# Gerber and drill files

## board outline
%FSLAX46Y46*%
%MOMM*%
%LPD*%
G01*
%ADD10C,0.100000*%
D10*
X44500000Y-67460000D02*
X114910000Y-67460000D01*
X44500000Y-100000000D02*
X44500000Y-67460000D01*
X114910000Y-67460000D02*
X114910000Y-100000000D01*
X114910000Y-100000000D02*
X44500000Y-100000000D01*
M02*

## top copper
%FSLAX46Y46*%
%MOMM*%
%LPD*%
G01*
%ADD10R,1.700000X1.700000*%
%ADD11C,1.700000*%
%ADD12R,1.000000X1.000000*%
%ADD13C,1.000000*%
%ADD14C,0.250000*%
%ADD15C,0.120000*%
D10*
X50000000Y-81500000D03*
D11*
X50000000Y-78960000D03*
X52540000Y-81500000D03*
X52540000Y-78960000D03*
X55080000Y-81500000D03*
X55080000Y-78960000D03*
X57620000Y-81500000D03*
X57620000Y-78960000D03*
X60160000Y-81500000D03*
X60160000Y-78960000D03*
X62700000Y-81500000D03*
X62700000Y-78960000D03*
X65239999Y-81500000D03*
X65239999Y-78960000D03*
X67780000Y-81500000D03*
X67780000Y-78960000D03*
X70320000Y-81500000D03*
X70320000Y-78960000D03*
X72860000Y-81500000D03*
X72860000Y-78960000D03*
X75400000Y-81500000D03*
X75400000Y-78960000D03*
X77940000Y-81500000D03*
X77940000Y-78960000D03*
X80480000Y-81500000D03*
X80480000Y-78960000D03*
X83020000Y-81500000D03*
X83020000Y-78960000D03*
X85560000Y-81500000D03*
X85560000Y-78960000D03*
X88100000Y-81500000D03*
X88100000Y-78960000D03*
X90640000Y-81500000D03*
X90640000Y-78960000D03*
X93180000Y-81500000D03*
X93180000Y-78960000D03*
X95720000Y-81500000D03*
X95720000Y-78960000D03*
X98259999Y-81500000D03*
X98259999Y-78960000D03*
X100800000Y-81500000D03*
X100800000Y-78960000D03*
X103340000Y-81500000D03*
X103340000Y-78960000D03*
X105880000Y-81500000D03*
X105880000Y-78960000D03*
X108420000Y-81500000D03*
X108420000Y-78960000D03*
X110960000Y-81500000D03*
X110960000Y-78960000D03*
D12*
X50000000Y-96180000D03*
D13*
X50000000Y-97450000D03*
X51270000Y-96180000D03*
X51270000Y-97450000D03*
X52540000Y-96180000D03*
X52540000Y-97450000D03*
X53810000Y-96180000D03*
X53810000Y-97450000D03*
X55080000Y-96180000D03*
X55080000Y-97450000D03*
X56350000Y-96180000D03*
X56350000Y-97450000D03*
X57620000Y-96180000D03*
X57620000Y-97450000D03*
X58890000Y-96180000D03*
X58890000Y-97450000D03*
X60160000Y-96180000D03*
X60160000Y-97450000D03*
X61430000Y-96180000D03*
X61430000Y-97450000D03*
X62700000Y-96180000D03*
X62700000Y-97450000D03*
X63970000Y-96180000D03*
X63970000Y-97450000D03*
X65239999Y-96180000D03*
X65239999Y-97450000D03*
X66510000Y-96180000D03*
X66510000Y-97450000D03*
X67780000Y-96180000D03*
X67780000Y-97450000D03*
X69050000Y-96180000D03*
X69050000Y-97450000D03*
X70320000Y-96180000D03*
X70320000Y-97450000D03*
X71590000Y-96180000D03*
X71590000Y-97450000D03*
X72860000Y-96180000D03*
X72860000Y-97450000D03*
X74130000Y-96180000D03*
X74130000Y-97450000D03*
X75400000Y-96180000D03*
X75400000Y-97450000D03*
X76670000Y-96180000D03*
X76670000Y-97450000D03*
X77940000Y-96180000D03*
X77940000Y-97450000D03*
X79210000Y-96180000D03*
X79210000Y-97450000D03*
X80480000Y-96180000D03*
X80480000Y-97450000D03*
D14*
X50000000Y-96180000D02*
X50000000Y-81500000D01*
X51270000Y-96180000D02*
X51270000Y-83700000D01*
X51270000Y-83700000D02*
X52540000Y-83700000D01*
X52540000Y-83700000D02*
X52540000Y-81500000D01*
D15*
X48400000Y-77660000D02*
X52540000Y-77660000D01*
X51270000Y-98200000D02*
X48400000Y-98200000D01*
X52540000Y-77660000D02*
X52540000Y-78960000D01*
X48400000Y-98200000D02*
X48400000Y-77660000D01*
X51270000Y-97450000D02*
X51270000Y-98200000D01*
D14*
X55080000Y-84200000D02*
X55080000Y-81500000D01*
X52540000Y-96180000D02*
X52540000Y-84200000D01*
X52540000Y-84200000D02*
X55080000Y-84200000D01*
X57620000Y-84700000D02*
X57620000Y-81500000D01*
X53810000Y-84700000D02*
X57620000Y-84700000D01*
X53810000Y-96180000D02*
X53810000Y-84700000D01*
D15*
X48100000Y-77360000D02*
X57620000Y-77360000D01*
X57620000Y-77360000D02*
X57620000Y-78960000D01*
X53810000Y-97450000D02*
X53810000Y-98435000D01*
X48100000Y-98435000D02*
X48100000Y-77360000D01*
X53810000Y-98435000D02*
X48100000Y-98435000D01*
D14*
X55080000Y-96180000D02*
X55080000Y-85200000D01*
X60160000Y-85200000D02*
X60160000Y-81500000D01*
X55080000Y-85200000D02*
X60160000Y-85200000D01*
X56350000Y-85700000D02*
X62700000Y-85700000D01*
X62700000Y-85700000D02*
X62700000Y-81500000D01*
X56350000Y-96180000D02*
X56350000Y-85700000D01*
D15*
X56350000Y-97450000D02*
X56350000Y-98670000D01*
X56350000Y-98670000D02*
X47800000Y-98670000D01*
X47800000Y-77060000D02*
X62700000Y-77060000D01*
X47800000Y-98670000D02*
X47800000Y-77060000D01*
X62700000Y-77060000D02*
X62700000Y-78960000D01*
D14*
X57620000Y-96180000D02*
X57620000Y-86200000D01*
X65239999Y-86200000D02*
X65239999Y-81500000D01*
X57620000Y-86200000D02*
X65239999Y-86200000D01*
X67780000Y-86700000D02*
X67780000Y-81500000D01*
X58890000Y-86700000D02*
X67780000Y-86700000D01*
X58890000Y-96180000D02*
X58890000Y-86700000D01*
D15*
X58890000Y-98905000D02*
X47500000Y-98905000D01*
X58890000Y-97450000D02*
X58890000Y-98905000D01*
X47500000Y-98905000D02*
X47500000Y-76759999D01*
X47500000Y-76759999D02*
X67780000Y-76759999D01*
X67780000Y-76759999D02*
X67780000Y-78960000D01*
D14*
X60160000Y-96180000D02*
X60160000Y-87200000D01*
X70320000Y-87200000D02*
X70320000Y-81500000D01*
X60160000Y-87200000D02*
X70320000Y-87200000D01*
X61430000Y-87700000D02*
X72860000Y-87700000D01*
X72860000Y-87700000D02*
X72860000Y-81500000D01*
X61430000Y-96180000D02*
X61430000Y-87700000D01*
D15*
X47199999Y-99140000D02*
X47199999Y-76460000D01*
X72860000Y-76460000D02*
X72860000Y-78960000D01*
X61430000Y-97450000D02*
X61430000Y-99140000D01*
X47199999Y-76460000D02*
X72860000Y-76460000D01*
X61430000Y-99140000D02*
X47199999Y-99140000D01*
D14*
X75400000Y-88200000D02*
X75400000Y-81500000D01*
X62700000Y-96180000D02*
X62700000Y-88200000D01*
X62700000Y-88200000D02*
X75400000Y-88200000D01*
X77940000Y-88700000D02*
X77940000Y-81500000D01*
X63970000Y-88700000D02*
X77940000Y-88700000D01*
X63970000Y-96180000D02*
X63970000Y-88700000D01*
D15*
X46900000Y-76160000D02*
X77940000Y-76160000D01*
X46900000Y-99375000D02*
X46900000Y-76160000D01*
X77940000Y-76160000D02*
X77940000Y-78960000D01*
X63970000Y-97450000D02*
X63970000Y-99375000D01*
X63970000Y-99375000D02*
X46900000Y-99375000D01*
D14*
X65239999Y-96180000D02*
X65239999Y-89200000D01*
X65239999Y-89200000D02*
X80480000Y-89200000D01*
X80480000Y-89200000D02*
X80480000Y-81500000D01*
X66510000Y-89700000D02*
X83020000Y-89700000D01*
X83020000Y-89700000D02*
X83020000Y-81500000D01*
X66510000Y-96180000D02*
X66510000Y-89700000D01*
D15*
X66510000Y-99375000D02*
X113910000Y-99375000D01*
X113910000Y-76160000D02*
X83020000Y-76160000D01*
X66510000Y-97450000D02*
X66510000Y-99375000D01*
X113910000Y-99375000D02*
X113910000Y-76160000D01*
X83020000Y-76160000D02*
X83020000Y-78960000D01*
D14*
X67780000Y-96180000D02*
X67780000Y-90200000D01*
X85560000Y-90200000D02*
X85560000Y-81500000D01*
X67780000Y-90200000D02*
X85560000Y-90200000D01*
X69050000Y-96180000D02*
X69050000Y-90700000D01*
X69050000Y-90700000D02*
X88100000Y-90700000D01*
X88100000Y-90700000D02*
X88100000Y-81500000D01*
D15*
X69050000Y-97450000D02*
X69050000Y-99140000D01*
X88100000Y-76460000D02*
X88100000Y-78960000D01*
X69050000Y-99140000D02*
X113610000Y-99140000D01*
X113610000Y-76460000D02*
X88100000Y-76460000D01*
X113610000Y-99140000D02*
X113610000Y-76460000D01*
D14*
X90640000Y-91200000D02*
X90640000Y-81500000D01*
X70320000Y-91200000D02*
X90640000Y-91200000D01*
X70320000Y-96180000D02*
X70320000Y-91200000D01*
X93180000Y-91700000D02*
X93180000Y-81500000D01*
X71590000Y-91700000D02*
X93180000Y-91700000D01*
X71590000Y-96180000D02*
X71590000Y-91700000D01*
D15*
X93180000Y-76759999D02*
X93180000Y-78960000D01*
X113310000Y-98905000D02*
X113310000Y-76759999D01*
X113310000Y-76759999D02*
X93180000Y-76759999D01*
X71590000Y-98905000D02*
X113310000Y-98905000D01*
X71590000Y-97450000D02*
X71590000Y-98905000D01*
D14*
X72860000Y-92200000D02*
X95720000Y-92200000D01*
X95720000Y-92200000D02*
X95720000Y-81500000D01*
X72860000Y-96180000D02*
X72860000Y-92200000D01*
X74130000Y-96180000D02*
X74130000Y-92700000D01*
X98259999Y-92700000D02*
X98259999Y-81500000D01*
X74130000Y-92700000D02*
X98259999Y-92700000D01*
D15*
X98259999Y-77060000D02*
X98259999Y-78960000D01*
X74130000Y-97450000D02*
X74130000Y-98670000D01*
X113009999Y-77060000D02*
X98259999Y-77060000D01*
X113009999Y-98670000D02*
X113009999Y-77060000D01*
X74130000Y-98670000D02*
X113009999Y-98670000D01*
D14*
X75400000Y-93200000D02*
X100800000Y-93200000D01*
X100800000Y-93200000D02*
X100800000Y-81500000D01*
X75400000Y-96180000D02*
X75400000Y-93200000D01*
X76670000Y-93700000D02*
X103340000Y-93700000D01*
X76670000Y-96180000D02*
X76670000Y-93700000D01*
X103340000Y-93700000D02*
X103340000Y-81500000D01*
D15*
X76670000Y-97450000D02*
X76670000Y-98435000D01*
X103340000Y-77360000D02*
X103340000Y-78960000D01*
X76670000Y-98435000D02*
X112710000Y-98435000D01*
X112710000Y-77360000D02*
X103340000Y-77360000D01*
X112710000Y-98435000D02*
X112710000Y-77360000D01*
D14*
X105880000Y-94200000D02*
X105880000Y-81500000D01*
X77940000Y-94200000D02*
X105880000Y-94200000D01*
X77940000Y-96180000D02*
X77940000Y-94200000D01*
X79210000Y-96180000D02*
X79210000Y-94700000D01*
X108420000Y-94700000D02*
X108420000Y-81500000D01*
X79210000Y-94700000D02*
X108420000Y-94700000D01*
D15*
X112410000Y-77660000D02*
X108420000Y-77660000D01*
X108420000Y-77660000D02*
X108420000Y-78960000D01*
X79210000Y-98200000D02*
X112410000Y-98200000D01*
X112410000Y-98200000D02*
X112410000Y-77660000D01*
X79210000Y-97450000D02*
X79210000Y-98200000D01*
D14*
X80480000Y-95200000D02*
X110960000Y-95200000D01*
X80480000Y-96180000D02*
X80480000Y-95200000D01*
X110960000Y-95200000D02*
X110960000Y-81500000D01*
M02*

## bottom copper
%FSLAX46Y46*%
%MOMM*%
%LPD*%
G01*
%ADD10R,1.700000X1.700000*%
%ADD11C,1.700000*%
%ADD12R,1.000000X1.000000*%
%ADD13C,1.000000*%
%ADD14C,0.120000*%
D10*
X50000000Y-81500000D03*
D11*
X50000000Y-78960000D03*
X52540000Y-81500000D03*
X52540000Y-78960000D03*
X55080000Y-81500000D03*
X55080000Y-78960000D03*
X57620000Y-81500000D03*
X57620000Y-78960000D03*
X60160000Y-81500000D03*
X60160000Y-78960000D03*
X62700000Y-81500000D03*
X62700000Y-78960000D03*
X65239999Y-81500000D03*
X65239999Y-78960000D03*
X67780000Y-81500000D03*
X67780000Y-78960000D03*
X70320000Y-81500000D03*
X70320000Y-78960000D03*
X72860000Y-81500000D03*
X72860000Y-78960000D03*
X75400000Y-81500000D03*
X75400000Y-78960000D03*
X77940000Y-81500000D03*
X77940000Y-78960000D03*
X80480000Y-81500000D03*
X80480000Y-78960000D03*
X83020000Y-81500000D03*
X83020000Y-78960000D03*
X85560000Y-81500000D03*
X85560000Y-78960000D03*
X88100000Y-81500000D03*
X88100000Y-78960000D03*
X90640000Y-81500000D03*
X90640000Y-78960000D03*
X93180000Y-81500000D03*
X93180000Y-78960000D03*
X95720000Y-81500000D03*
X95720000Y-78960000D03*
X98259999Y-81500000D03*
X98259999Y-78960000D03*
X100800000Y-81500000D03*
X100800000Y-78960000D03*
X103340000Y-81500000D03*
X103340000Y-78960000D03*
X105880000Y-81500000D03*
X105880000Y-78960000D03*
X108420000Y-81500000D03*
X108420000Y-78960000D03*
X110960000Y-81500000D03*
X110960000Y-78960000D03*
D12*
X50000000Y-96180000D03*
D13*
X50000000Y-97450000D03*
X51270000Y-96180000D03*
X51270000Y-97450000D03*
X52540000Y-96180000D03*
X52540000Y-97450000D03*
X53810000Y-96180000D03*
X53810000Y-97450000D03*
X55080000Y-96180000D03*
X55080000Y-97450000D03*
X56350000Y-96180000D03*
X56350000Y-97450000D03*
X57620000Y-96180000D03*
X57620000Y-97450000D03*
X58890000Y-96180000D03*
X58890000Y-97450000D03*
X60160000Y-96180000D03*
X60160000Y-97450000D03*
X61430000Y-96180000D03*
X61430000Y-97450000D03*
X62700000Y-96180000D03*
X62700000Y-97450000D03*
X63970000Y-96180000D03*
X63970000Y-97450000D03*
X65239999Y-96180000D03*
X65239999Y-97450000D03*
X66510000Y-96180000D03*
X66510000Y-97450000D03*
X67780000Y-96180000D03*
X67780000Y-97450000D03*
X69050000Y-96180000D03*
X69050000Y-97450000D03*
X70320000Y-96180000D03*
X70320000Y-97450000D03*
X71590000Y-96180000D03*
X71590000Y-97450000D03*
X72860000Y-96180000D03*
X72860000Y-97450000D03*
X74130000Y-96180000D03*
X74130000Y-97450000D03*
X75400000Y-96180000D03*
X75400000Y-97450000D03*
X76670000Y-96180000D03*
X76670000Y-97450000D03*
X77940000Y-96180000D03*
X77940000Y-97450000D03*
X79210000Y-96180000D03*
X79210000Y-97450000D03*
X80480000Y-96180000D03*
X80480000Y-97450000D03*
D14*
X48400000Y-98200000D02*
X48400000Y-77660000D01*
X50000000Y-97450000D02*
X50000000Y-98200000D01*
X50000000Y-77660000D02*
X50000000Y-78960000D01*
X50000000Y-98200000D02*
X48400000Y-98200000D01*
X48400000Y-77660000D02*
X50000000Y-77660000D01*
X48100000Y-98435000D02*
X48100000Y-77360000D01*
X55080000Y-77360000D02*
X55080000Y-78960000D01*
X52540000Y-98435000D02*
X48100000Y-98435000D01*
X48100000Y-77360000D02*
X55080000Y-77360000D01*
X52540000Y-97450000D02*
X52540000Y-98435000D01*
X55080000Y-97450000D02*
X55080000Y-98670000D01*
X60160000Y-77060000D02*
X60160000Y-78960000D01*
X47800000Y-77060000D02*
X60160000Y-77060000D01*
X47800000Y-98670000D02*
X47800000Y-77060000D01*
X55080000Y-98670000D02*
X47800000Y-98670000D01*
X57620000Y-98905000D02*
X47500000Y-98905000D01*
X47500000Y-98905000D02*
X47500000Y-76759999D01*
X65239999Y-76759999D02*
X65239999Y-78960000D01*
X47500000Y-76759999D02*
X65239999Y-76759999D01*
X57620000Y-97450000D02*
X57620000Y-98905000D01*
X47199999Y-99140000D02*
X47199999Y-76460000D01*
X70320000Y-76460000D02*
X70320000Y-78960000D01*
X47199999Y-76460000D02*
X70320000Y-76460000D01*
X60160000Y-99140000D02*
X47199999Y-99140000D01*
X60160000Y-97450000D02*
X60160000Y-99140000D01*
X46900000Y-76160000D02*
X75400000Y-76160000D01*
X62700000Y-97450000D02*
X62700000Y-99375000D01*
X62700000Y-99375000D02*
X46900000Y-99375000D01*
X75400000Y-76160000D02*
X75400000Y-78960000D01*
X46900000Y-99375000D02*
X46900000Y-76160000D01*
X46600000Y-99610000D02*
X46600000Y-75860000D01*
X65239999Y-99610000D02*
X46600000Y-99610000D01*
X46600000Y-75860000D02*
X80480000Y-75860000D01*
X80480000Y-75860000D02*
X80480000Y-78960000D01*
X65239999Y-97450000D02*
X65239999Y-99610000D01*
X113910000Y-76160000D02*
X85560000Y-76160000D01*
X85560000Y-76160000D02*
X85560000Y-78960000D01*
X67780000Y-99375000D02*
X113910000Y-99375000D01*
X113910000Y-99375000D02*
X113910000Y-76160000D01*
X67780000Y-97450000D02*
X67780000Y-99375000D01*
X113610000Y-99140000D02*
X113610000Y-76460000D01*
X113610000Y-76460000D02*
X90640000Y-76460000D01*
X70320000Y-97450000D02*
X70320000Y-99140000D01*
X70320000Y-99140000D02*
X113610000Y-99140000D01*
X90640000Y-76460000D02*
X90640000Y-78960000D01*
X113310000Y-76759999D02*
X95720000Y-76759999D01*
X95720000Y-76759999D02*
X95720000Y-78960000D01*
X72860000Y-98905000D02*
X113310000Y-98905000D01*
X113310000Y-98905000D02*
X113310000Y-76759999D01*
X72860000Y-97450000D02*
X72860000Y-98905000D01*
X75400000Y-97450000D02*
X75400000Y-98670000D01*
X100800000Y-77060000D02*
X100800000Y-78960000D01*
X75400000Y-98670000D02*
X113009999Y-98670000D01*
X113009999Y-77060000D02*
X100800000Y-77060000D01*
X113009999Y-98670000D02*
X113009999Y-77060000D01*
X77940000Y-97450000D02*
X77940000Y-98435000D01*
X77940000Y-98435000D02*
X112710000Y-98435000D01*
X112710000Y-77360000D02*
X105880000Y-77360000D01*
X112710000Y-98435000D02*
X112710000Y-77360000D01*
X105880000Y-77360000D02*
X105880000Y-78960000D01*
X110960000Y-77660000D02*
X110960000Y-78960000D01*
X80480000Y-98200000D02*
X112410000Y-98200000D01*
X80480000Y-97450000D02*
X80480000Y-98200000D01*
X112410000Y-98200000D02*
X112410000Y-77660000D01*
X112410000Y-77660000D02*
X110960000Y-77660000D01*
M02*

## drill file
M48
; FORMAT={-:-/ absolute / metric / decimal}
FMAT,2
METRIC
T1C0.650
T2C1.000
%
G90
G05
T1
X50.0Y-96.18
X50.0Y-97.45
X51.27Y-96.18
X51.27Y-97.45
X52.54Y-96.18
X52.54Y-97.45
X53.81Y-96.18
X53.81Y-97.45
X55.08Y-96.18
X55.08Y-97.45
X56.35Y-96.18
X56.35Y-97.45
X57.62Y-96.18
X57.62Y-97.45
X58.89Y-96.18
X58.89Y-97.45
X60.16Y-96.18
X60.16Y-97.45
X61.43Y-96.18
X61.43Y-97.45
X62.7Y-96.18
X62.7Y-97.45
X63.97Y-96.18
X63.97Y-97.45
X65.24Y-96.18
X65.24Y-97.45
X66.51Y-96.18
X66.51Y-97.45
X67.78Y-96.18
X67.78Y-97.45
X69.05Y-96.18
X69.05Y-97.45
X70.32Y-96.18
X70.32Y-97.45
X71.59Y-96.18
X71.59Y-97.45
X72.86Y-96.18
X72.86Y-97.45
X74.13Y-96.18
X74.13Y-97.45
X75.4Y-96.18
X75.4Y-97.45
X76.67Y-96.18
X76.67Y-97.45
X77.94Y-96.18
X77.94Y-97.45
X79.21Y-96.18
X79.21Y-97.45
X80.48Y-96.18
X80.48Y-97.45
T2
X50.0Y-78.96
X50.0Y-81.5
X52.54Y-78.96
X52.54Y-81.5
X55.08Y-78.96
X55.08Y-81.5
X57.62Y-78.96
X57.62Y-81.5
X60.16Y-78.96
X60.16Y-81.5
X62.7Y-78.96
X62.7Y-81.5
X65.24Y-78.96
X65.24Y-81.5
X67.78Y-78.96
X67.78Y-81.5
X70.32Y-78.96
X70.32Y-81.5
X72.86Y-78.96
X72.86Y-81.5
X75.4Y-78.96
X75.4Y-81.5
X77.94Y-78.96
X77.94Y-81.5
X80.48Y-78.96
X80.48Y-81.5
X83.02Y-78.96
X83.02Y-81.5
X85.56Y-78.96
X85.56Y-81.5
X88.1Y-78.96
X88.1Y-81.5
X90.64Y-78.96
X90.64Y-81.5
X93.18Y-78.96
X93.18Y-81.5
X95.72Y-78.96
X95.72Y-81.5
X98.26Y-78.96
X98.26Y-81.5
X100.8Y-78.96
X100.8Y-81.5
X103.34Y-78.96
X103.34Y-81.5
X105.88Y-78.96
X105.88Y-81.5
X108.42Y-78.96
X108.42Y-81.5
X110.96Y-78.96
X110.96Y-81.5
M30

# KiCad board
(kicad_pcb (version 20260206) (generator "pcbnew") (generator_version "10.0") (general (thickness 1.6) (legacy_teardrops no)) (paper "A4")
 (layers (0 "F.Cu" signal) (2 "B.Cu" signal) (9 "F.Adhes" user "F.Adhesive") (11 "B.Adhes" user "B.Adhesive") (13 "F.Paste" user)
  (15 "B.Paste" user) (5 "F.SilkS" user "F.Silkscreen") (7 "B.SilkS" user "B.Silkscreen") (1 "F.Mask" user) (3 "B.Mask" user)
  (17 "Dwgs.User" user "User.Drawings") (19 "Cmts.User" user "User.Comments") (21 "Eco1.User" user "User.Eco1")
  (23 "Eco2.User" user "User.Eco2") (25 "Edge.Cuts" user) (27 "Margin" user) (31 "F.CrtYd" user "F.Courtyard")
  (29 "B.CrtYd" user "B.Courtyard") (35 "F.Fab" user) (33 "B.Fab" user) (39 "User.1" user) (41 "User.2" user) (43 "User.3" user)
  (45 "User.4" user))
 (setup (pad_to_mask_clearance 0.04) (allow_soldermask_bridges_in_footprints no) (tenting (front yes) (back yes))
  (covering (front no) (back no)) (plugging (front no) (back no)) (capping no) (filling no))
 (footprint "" (layer "F.Cu") (at 80.48 80.229999)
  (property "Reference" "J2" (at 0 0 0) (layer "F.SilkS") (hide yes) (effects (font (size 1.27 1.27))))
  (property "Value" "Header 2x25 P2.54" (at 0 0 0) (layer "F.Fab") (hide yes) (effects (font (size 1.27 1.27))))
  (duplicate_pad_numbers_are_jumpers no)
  (pad "1" thru_hole rect (at -30.48 1.270001) (size 1.7 1.7) (drill 1) (layers "*.Cu" "*.Mask") (remove_unused_layers no) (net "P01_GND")
   (thermal_bridge_angle 45))
  (pad "2" thru_hole circle (at -30.48 -1.269999) (size 1.7 1.7) (drill 1) (layers "*.Cu" "*.Mask") (remove_unused_layers no) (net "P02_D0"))
  (pad "3" thru_hole circle (at -27.94 1.270001) (size 1.7 1.7) (drill 1) (layers "*.Cu" "*.Mask") (remove_unused_layers no) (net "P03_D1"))
  (pad "4" thru_hole circle (at -27.94 -1.269999) (size 1.7 1.7) (drill 1) (layers "*.Cu" "*.Mask") (remove_unused_layers no) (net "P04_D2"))
  (pad "5" thru_hole circle (at -25.4 1.270001) (size 1.7 1.7) (drill 1) (layers "*.Cu" "*.Mask") (remove_unused_layers no) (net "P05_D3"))
  (pad "6" thru_hole circle (at -25.4 -1.269999) (size 1.7 1.7) (drill 1) (layers "*.Cu" "*.Mask") (remove_unused_layers no) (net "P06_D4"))
  (pad "7" thru_hole circle (at -22.86 1.270001) (size 1.7 1.7) (drill 1) (layers "*.Cu" "*.Mask") (remove_unused_layers no) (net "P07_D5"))
  (pad "8" thru_hole circle (at -22.86 -1.269999) (size 1.7 1.7) (drill 1) (layers "*.Cu" "*.Mask") (remove_unused_layers no) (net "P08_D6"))
  (pad "9" thru_hole circle (at -20.32 1.270001) (size 1.7 1.7) (drill 1) (layers "*.Cu" "*.Mask") (remove_unused_layers no) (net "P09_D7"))
  (pad "10" thru_hole circle (at -20.32 -1.269999) (size 1.7 1.7) (drill 1) (layers "*.Cu" "*.Mask") (remove_unused_layers no)
   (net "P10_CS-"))
  (pad "11" thru_hole circle (at -17.78 1.270001) (size 1.7 1.7) (drill 1) (layers "*.Cu" "*.Mask") (remove_unused_layers no)
   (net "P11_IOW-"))
  (pad "12" thru_hole circle (at -17.78 -1.269999) (size 1.7 1.7) (drill 1) (layers "*.Cu" "*.Mask") (remove_unused_layers no)
   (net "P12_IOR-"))
  (pad "13" thru_hole circle (at -15.240001 1.270001) (size 1.7 1.7) (drill 1) (layers "*.Cu" "*.Mask") (remove_unused_layers no)
   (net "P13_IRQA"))
  (pad "14" thru_hole circle (at -15.240001 -1.269999) (size 1.7 1.7) (drill 1) (layers "*.Cu" "*.Mask") (remove_unused_layers no)
   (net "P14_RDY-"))
  (pad "15" thru_hole circle (at -12.7 1.270001) (size 1.7 1.7) (drill 1) (layers "*.Cu" "*.Mask") (remove_unused_layers no) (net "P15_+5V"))
  (pad "16" thru_hole circle (at -12.7 -1.269999) (size 1.7 1.7) (drill 1) (layers "*.Cu" "*.Mask") (remove_unused_layers no)
   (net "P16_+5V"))
  (pad "17" thru_hole circle (at -10.16 1.270001) (size 1.7 1.7) (drill 1) (layers "*.Cu" "*.Mask") (remove_unused_layers no)
   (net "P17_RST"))
  (pad "18" thru_hole circle (at -10.16 -1.269999) (size 1.7 1.7) (drill 1) (layers "*.Cu" "*.Mask") (remove_unused_layers no)
   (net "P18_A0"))
  (pad "19" thru_hole circle (at -7.62 1.270001) (size 1.7 1.7) (drill 1) (layers "*.Cu" "*.Mask") (remove_unused_layers no) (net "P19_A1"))
  (pad "20" thru_hole circle (at -7.62 -1.269999) (size 1.7 1.7) (drill 1) (layers "*.Cu" "*.Mask") (remove_unused_layers no) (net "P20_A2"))
  (pad "21" thru_hole circle (at -5.08 1.270001) (size 1.7 1.7) (drill 1) (layers "*.Cu" "*.Mask") (remove_unused_layers no) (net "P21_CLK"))
  (pad "22" thru_hole circle (at -5.08 -1.269999) (size 1.7 1.7) (drill 1) (layers "*.Cu" "*.Mask") (remove_unused_layers no)
   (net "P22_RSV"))
  (pad "23" thru_hole circle (at -2.54 1.270001) (size 1.7 1.7) (drill 1) (layers "*.Cu" "*.Mask") (remove_unused_layers no)
   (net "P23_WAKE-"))
  (pad "24" thru_hole circle (at -2.54 -1.269999) (size 1.7 1.7) (drill 1) (layers "*.Cu" "*.Mask") (remove_unused_layers no)
   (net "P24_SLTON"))
  (pad "25" thru_hole circle (at 0 1.270001) (size 1.7 1.7) (drill 1) (layers "*.Cu" "*.Mask") (remove_unused_layers no) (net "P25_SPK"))
  (pad "26" thru_hole circle (at 0 -1.269999) (size 1.7 1.7) (drill 1) (layers "*.Cu" "*.Mask") (remove_unused_layers no) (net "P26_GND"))
  (pad "27" thru_hole circle (at 2.54 1.270001) (size 1.7 1.7) (drill 1) (layers "*.Cu" "*.Mask") (remove_unused_layers no) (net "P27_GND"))
  (pad "28" thru_hole circle (at 2.54 -1.269999) (size 1.7 1.7) (drill 1) (layers "*.Cu" "*.Mask") (remove_unused_layers no) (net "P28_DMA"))
  (pad "29" thru_hole circle (at 5.08 1.270001) (size 1.7 1.7) (drill 1) (layers "*.Cu" "*.Mask") (remove_unused_layers no) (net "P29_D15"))
  (pad "30" thru_hole circle (at 5.08 -1.269999) (size 1.7 1.7) (drill 1) (layers "*.Cu" "*.Mask") (remove_unused_layers no) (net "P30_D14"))
  (pad "31" thru_hole circle (at 7.62 1.270001) (size 1.7 1.7) (drill 1) (layers "*.Cu" "*.Mask") (remove_unused_layers no) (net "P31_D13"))
  (pad "32" thru_hole circle (at 7.62 -1.269999) (size 1.7 1.7) (drill 1) (layers "*.Cu" "*.Mask") (remove_unused_layers no) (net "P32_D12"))
  (pad "33" thru_hole circle (at 10.16 1.270001) (size 1.7 1.7) (drill 1) (layers "*.Cu" "*.Mask") (remove_unused_layers no) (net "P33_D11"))
  (pad "34" thru_hole circle (at 10.16 -1.269999) (size 1.7 1.7) (drill 1) (layers "*.Cu" "*.Mask") (remove_unused_layers no)
   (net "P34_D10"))
  (pad "35" thru_hole circle (at 12.7 1.270001) (size 1.7 1.7) (drill 1) (layers "*.Cu" "*.Mask") (remove_unused_layers no) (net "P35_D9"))
  (pad "36" thru_hole circle (at 12.7 -1.269999) (size 1.7 1.7) (drill 1) (layers "*.Cu" "*.Mask") (remove_unused_layers no) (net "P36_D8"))
  (pad "37" thru_hole circle (at 15.24 1.270001) (size 1.7 1.7) (drill 1) (layers "*.Cu" "*.Mask") (remove_unused_layers no) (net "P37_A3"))
  (pad "38" thru_hole circle (at 15.24 -1.269999) (size 1.7 1.7) (drill 1) (layers "*.Cu" "*.Mask") (remove_unused_layers no) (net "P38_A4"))
  (pad "39" thru_hole circle (at 17.779999 1.270001) (size 1.7 1.7) (drill 1) (layers "*.Cu" "*.Mask") (remove_unused_layers no)
   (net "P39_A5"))
  (pad "40" thru_hole circle (at 17.779999 -1.269999) (size 1.7 1.7) (drill 1) (layers "*.Cu" "*.Mask") (remove_unused_layers no)
   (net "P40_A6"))
  (pad "41" thru_hole circle (at 20.32 1.270001) (size 1.7 1.7) (drill 1) (layers "*.Cu" "*.Mask") (remove_unused_layers no) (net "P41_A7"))
  (pad "42" thru_hole circle (at 20.32 -1.269999) (size 1.7 1.7) (drill 1) (layers "*.Cu" "*.Mask") (remove_unused_layers no) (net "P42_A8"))
  (pad "43" thru_hole circle (at 22.86 1.270001) (size 1.7 1.7) (drill 1) (layers "*.Cu" "*.Mask") (remove_unused_layers no) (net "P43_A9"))
  (pad "44" thru_hole circle (at 22.86 -1.269999) (size 1.7 1.7) (drill 1) (layers "*.Cu" "*.Mask") (remove_unused_layers no)
   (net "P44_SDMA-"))
  (pad "45" thru_hole circle (at 25.4 1.270001) (size 1.7 1.7) (drill 1) (layers "*.Cu" "*.Mask") (remove_unused_layers no) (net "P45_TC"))
  (pad "46" thru_hole circle (at 25.4 -1.269999) (size 1.7 1.7) (drill 1) (layers "*.Cu" "*.Mask") (remove_unused_layers no)
   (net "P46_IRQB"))
  (pad "47" thru_hole circle (at 27.94 1.270001) (size 1.7 1.7) (drill 1) (layers "*.Cu" "*.Mask") (remove_unused_layers no)
   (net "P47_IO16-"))
  (pad "48" thru_hole circle (at 27.94 -1.269999) (size 1.7 1.7) (drill 1) (layers "*.Cu" "*.Mask") (remove_unused_layers no)
   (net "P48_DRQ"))
  (pad "49" thru_hole circle (at 30.48 1.270001) (size 1.7 1.7) (drill 1) (layers "*.Cu" "*.Mask") (remove_unused_layers no)
   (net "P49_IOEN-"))
  (pad "50" thru_hole circle (at 30.48 -1.269999) (size 1.7 1.7) (drill 1) (layers "*.Cu" "*.Mask") (remove_unused_layers no)
   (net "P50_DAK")))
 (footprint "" (layer "F.Cu") (at 65.239999 96.815)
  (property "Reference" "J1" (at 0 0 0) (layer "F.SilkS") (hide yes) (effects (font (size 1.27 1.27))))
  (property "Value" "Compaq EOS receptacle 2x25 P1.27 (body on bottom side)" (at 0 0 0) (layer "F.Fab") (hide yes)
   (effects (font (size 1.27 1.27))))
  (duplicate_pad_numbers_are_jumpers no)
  (pad "1" thru_hole rect (at -15.239999 -0.635) (size 1 1) (drill 0.65) (layers "*.Cu" "*.Mask") (remove_unused_layers no) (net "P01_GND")
   (thermal_bridge_angle 45))
  (pad "2" thru_hole circle (at -15.239999 0.635) (size 1 1) (drill 0.65) (layers "*.Cu" "*.Mask") (remove_unused_layers no) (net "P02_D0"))
  (pad "3" thru_hole circle (at -13.969999 -0.635) (size 1 1) (drill 0.65) (layers "*.Cu" "*.Mask") (remove_unused_layers no) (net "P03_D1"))
  (pad "4" thru_hole circle (at -13.969999 0.635) (size 1 1) (drill 0.65) (layers "*.Cu" "*.Mask") (remove_unused_layers no) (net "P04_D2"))
  (pad "5" thru_hole circle (at -12.699999 -0.635) (size 1 1) (drill 0.65) (layers "*.Cu" "*.Mask") (remove_unused_layers no) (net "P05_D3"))
  (pad "6" thru_hole circle (at -12.699999 0.635) (size 1 1) (drill 0.65) (layers "*.Cu" "*.Mask") (remove_unused_layers no) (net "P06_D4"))
  (pad "7" thru_hole circle (at -11.429999 -0.635) (size 1 1) (drill 0.65) (layers "*.Cu" "*.Mask") (remove_unused_layers no) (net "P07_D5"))
  (pad "8" thru_hole circle (at -11.429999 0.635) (size 1 1) (drill 0.65) (layers "*.Cu" "*.Mask") (remove_unused_layers no) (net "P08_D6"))
  (pad "9" thru_hole circle (at -10.159999 -0.635) (size 1 1) (drill 0.65) (layers "*.Cu" "*.Mask") (remove_unused_layers no) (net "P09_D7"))
  (pad "10" thru_hole circle (at -10.159999 0.635) (size 1 1) (drill 0.65) (layers "*.Cu" "*.Mask") (remove_unused_layers no)
   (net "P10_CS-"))
  (pad "11" thru_hole circle (at -8.889999 -0.635) (size 1 1) (drill 0.65) (layers "*.Cu" "*.Mask") (remove_unused_layers no)
   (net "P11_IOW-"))
  (pad "12" thru_hole circle (at -8.889999 0.635) (size 1 1) (drill 0.65) (layers "*.Cu" "*.Mask") (remove_unused_layers no)
   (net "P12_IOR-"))
  (pad "13" thru_hole circle (at -7.619999 -0.635) (size 1 1) (drill 0.65) (layers "*.Cu" "*.Mask") (remove_unused_layers no)
   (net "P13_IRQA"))
  (pad "14" thru_hole circle (at -7.619999 0.635) (size 1 1) (drill 0.65) (layers "*.Cu" "*.Mask") (remove_unused_layers no)
   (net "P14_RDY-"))
  (pad "15" thru_hole circle (at -6.349999 -0.635) (size 1 1) (drill 0.65) (layers "*.Cu" "*.Mask") (remove_unused_layers no)
   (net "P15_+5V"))
  (pad "16" thru_hole circle (at -6.349999 0.635) (size 1 1) (drill 0.65) (layers "*.Cu" "*.Mask") (remove_unused_layers no) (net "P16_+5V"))
  (pad "17" thru_hole circle (at -5.079999 -0.635) (size 1 1) (drill 0.65) (layers "*.Cu" "*.Mask") (remove_unused_layers no)
   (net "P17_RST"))
  (pad "18" thru_hole circle (at -5.079999 0.635) (size 1 1) (drill 0.65) (layers "*.Cu" "*.Mask") (remove_unused_layers no) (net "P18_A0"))
  (pad "19" thru_hole circle (at -3.809999 -0.635) (size 1 1) (drill 0.65) (layers "*.Cu" "*.Mask") (remove_unused_layers no) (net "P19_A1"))
  (pad "20" thru_hole circle (at -3.809999 0.635) (size 1 1) (drill 0.65) (layers "*.Cu" "*.Mask") (remove_unused_layers no) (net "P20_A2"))
  (pad "21" thru_hole circle (at -2.539999 -0.635) (size 1 1) (drill 0.65) (layers "*.Cu" "*.Mask") (remove_unused_layers no)
   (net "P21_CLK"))
  (pad "22" thru_hole circle (at -2.539999 0.635) (size 1 1) (drill 0.65) (layers "*.Cu" "*.Mask") (remove_unused_layers no) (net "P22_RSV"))
  (pad "23" thru_hole circle (at -1.269999 -0.635) (size 1 1) (drill 0.65) (layers "*.Cu" "*.Mask") (remove_unused_layers no)
   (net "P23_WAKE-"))
  (pad "24" thru_hole circle (at -1.269999 0.635) (size 1 1) (drill 0.65) (layers "*.Cu" "*.Mask") (remove_unused_layers no)
   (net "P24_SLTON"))
  (pad "25" thru_hole circle (at 0 -0.635) (size 1 1) (drill 0.65) (layers "*.Cu" "*.Mask") (remove_unused_layers no) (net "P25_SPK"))
  (pad "26" thru_hole circle (at 0 0.635) (size 1 1) (drill 0.65) (layers "*.Cu" "*.Mask") (remove_unused_layers no) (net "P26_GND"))
  (pad "27" thru_hole circle (at 1.270001 -0.635) (size 1 1) (drill 0.65) (layers "*.Cu" "*.Mask") (remove_unused_layers no) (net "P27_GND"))
  (pad "28" thru_hole circle (at 1.270001 0.635) (size 1 1) (drill 0.65) (layers "*.Cu" "*.Mask") (remove_unused_layers no) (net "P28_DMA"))
  (pad "29" thru_hole circle (at 2.540001 -0.635) (size 1 1) (drill 0.65) (layers "*.Cu" "*.Mask") (remove_unused_layers no) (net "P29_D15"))
  (pad "30" thru_hole circle (at 2.540001 0.635) (size 1 1) (drill 0.65) (layers "*.Cu" "*.Mask") (remove_unused_layers no) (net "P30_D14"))
  (pad "31" thru_hole circle (at 3.810001 -0.635) (size 1 1) (drill 0.65) (layers "*.Cu" "*.Mask") (remove_unused_layers no) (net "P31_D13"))
  (pad "32" thru_hole circle (at 3.810001 0.635) (size 1 1) (drill 0.65) (layers "*.Cu" "*.Mask") (remove_unused_layers no) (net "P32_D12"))
  (pad "33" thru_hole circle (at 5.080001 -0.635) (size 1 1) (drill 0.65) (layers "*.Cu" "*.Mask") (remove_unused_layers no) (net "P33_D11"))
  (pad "34" thru_hole circle (at 5.080001 0.635) (size 1 1) (drill 0.65) (layers "*.Cu" "*.Mask") (remove_unused_layers no) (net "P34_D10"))
  (pad "35" thru_hole circle (at 6.350001 -0.635) (size 1 1) (drill 0.65) (layers "*.Cu" "*.Mask") (remove_unused_layers no) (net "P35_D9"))
  (pad "36" thru_hole circle (at 6.350001 0.635) (size 1 1) (drill 0.65) (layers "*.Cu" "*.Mask") (remove_unused_layers no) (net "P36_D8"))
  (pad "37" thru_hole circle (at 7.620001 -0.635) (size 1 1) (drill 0.65) (layers "*.Cu" "*.Mask") (remove_unused_layers no) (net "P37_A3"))
  (pad "38" thru_hole circle (at 7.620001 0.635) (size 1 1) (drill 0.65) (layers "*.Cu" "*.Mask") (remove_unused_layers no) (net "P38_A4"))
  (pad "39" thru_hole circle (at 8.890001 -0.635) (size 1 1) (drill 0.65) (layers "*.Cu" "*.Mask") (remove_unused_layers no) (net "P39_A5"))
  (pad "40" thru_hole circle (at 8.890001 0.635) (size 1 1) (drill 0.65) (layers "*.Cu" "*.Mask") (remove_unused_layers no) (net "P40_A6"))
  (pad "41" thru_hole circle (at 10.160001 -0.635) (size 1 1) (drill 0.65) (layers "*.Cu" "*.Mask") (remove_unused_layers no) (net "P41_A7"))
  (pad "42" thru_hole circle (at 10.160001 0.635) (size 1 1) (drill 0.65) (layers "*.Cu" "*.Mask") (remove_unused_layers no) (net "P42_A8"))
  (pad "43" thru_hole circle (at 11.430001 -0.635) (size 1 1) (drill 0.65) (layers "*.Cu" "*.Mask") (remove_unused_layers no) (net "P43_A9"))
  (pad "44" thru_hole circle (at 11.430001 0.635) (size 1 1) (drill 0.65) (layers "*.Cu" "*.Mask") (remove_unused_layers no)
   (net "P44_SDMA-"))
  (pad "45" thru_hole circle (at 12.700001 -0.635) (size 1 1) (drill 0.65) (layers "*.Cu" "*.Mask") (remove_unused_layers no) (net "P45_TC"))
  (pad "46" thru_hole circle (at 12.700001 0.635) (size 1 1) (drill 0.65) (layers "*.Cu" "*.Mask") (remove_unused_layers no)
   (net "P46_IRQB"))
  (pad "47" thru_hole circle (at 13.970001 -0.635) (size 1 1) (drill 0.65) (layers "*.Cu" "*.Mask") (remove_unused_layers no)
   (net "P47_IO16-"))
  (pad "48" thru_hole circle (at 13.970001 0.635) (size 1 1) (drill 0.65) (layers "*.Cu" "*.Mask") (remove_unused_layers no) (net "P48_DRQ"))
  (pad "49" thru_hole circle (at 15.240001 -0.635) (size 1 1) (drill 0.65) (layers "*.Cu" "*.Mask") (remove_unused_layers no)
   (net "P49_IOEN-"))
  (pad "50" thru_hole circle (at 15.240001 0.635) (size 1 1) (drill 0.65) (layers "*.Cu" "*.Mask") (remove_unused_layers no) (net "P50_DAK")))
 (gr_line (start 44.5 67.46) (end 114.91 67.46) (stroke (width 0.1) (type default)) (layer "Edge.Cuts"))
 (gr_line (start 44.5 100) (end 44.5 67.46) (stroke (width 0.1) (type default)) (layer "Edge.Cuts"))
 (gr_line (start 114.91 67.46) (end 114.91 100) (stroke (width 0.1) (type default)) (layer "Edge.Cuts"))
 (gr_line (start 114.91 100) (end 44.5 100) (stroke (width 0.1) (type default)) (layer "Edge.Cuts"))
 (segment (start 50 96.18) (end 50 81.5) (width 0.25) (layer "F.Cu") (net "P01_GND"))
 (segment (start 48.4 98.2) (end 48.4 77.66) (width 0.12) (layer "B.Cu") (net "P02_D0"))
 (segment (start 50 97.45) (end 50 98.2) (width 0.12) (layer "B.Cu") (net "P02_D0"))
 (segment (start 50 77.66) (end 50 78.96) (width 0.12) (layer "B.Cu") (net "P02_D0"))
 (segment (start 50 98.2) (end 48.4 98.2) (width 0.12) (layer "B.Cu") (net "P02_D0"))
 (segment (start 48.4 77.66) (end 50 77.66) (width 0.12) (layer "B.Cu") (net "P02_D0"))
 (segment (start 51.27 96.18) (end 51.27 83.7) (width 0.25) (layer "F.Cu") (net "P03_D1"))
 (segment (start 51.27 83.7) (end 52.54 83.7) (width 0.25) (layer "F.Cu") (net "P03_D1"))
 (segment (start 52.54 83.7) (end 52.54 81.5) (width 0.25) (layer "F.Cu") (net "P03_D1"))
 (segment (start 48.4 77.66) (end 52.54 77.66) (width 0.12) (layer "F.Cu") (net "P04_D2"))
 (segment (start 51.27 98.2) (end 48.4 98.2) (width 0.12) (layer "F.Cu") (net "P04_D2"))
 (segment (start 52.54 77.66) (end 52.54 78.96) (width 0.12) (layer "F.Cu") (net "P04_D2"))
 (segment (start 48.4 98.2) (end 48.4 77.66) (width 0.12) (layer "F.Cu") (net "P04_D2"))
 (segment (start 51.27 97.45) (end 51.27 98.2) (width 0.12) (layer "F.Cu") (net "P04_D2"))
 (segment (start 55.08 84.2) (end 55.08 81.5) (width 0.25) (layer "F.Cu") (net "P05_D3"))
 (segment (start 52.54 96.18) (end 52.54 84.2) (width 0.25) (layer "F.Cu") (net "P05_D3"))
 (segment (start 52.54 84.2) (end 55.08 84.2) (width 0.25) (layer "F.Cu") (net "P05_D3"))
 (segment (start 48.1 98.435) (end 48.1 77.36) (width 0.12) (layer "B.Cu") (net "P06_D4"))
 (segment (start 55.08 77.36) (end 55.08 78.96) (width 0.12) (layer "B.Cu") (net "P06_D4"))
 (segment (start 52.54 98.435) (end 48.1 98.435) (width 0.12) (layer "B.Cu") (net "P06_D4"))
 (segment (start 48.1 77.36) (end 55.08 77.36) (width 0.12) (layer "B.Cu") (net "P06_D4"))
 (segment (start 52.54 97.45) (end 52.54 98.435) (width 0.12) (layer "B.Cu") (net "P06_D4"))
 (segment (start 57.62 84.7) (end 57.62 81.5) (width 0.25) (layer "F.Cu") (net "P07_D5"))
 (segment (start 53.81 84.7) (end 57.62 84.7) (width 0.25) (layer "F.Cu") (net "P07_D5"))
 (segment (start 53.81 96.18) (end 53.81 84.7) (width 0.25) (layer "F.Cu") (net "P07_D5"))
 (segment (start 48.1 77.36) (end 57.62 77.36) (width 0.12) (layer "F.Cu") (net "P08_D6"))
 (segment (start 57.62 77.36) (end 57.62 78.96) (width 0.12) (layer "F.Cu") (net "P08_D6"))
 (segment (start 53.81 97.45) (end 53.81 98.435) (width 0.12) (layer "F.Cu") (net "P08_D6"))
 (segment (start 48.1 98.435) (end 48.1 77.36) (width 0.12) (layer "F.Cu") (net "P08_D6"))
 (segment (start 53.81 98.435) (end 48.1 98.435) (width 0.12) (layer "F.Cu") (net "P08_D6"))
 (segment (start 55.08 96.18) (end 55.08 85.2) (width 0.25) (layer "F.Cu") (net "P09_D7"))
 (segment (start 60.16 85.2) (end 60.16 81.5) (width 0.25) (layer "F.Cu") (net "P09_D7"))
 (segment (start 55.08 85.2) (end 60.16 85.2) (width 0.25) (layer "F.Cu") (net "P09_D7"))
 (segment (start 55.08 97.45) (end 55.08 98.67) (width 0.12) (layer "B.Cu") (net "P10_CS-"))
 (segment (start 60.16 77.06) (end 60.16 78.96) (width 0.12) (layer "B.Cu") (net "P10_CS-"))
 (segment (start 47.8 77.06) (end 60.16 77.06) (width 0.12) (layer "B.Cu") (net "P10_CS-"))
 (segment (start 47.8 98.67) (end 47.8 77.06) (width 0.12) (layer "B.Cu") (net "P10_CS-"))
 (segment (start 55.08 98.67) (end 47.8 98.67) (width 0.12) (layer "B.Cu") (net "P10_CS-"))
 (segment (start 56.35 85.7) (end 62.7 85.7) (width 0.25) (layer "F.Cu") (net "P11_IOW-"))
 (segment (start 62.7 85.7) (end 62.7 81.5) (width 0.25) (layer "F.Cu") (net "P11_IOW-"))
 (segment (start 56.35 96.18) (end 56.35 85.7) (width 0.25) (layer "F.Cu") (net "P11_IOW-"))
 (segment (start 56.35 97.45) (end 56.35 98.67) (width 0.12) (layer "F.Cu") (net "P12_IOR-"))
 (segment (start 56.35 98.67) (end 47.8 98.67) (width 0.12) (layer "F.Cu") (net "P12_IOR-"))
 (segment (start 47.8 77.06) (end 62.7 77.06) (width 0.12) (layer "F.Cu") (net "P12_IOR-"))
 (segment (start 47.8 98.67) (end 47.8 77.06) (width 0.12) (layer "F.Cu") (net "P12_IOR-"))
 (segment (start 62.7 77.06) (end 62.7 78.96) (width 0.12) (layer "F.Cu") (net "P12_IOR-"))
 (segment (start 57.62 96.18) (end 57.62 86.2) (width 0.25) (layer "F.Cu") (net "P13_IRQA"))
 (segment (start 65.239999 86.2) (end 65.239999 81.5) (width 0.25) (layer "F.Cu") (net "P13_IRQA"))
 (segment (start 57.62 86.2) (end 65.239999 86.2) (width 0.25) (layer "F.Cu") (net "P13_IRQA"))
 (segment (start 57.62 98.905) (end 47.5 98.905) (width 0.12) (layer "B.Cu") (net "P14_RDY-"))
 (segment (start 47.5 98.905) (end 47.5 76.759999) (width 0.12) (layer "B.Cu") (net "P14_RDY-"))
 (segment (start 65.239999 76.759999) (end 65.239999 78.96) (width 0.12) (layer "B.Cu") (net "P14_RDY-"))
 (segment (start 47.5 76.759999) (end 65.239999 76.759999) (width 0.12) (layer "B.Cu") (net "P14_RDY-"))
 (segment (start 57.62 97.45) (end 57.62 98.905) (width 0.12) (layer "B.Cu") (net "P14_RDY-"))
 (segment (start 67.78 86.7) (end 67.78 81.5) (width 0.25) (layer "F.Cu") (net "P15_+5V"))
 (segment (start 58.89 86.7) (end 67.78 86.7) (width 0.25) (layer "F.Cu") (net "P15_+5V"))
 (segment (start 58.89 96.18) (end 58.89 86.7) (width 0.25) (layer "F.Cu") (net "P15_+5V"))
 (segment (start 58.89 98.905) (end 47.5 98.905) (width 0.12) (layer "F.Cu") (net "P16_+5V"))
 (segment (start 58.89 97.45) (end 58.89 98.905) (width 0.12) (layer "F.Cu") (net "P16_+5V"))
 (segment (start 47.5 98.905) (end 47.5 76.759999) (width 0.12) (layer "F.Cu") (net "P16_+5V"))
 (segment (start 47.5 76.759999) (end 67.78 76.759999) (width 0.12) (layer "F.Cu") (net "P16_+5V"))
 (segment (start 67.78 76.759999) (end 67.78 78.96) (width 0.12) (layer "F.Cu") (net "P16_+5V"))
 (segment (start 60.16 96.18) (end 60.16 87.2) (width 0.25) (layer "F.Cu") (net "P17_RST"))
 (segment (start 70.32 87.2) (end 70.32 81.5) (width 0.25) (layer "F.Cu") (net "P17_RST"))
 (segment (start 60.16 87.2) (end 70.32 87.2) (width 0.25) (layer "F.Cu") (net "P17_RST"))
 (segment (start 47.199999 99.14) (end 47.199999 76.46) (width 0.12) (layer "B.Cu") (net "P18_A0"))
 (segment (start 70.32 76.46) (end 70.32 78.96) (width 0.12) (layer "B.Cu") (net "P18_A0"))
 (segment (start 47.199999 76.46) (end 70.32 76.46) (width 0.12) (layer "B.Cu") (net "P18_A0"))
 (segment (start 60.16 99.14) (end 47.199999 99.14) (width 0.12) (layer "B.Cu") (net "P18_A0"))
 (segment (start 60.16 97.45) (end 60.16 99.14) (width 0.12) (layer "B.Cu") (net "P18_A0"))
 (segment (start 61.43 87.7) (end 72.86 87.7) (width 0.25) (layer "F.Cu") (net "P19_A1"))
 (segment (start 72.86 87.7) (end 72.86 81.5) (width 0.25) (layer "F.Cu") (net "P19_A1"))
 (segment (start 61.43 96.18) (end 61.43 87.7) (width 0.25) (layer "F.Cu") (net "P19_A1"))
 (segment (start 47.199999 99.14) (end 47.199999 76.46) (width 0.12) (layer "F.Cu") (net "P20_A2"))
 (segment (start 72.86 76.46) (end 72.86 78.96) (width 0.12) (layer "F.Cu") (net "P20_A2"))
 (segment (start 61.43 97.45) (end 61.43 99.14) (width 0.12) (layer "F.Cu") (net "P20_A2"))
 (segment (start 47.199999 76.46) (end 72.86 76.46) (width 0.12) (layer "F.Cu") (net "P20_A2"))
 (segment (start 61.43 99.14) (end 47.199999 99.14) (width 0.12) (layer "F.Cu") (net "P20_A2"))
 (segment (start 75.4 88.2) (end 75.4 81.5) (width 0.25) (layer "F.Cu") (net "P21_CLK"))
 (segment (start 62.7 96.18) (end 62.7 88.2) (width 0.25) (layer "F.Cu") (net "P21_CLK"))
 (segment (start 62.7 88.2) (end 75.4 88.2) (width 0.25) (layer "F.Cu") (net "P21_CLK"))
 (segment (start 46.9 76.16) (end 75.4 76.16) (width 0.12) (layer "B.Cu") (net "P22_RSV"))
 (segment (start 62.7 97.45) (end 62.7 99.375) (width 0.12) (layer "B.Cu") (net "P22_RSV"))
 (segment (start 62.7 99.375) (end 46.9 99.375) (width 0.12) (layer "B.Cu") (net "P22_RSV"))
 (segment (start 75.4 76.16) (end 75.4 78.96) (width 0.12) (layer "B.Cu") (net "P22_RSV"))
 (segment (start 46.9 99.375) (end 46.9 76.16) (width 0.12) (layer "B.Cu") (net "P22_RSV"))
 (segment (start 77.94 88.7) (end 77.94 81.5) (width 0.25) (layer "F.Cu") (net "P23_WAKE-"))
 (segment (start 63.97 88.7) (end 77.94 88.7) (width 0.25) (layer "F.Cu") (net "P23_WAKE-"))
 (segment (start 63.97 96.18) (end 63.97 88.7) (width 0.25) (layer "F.Cu") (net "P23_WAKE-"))
 (segment (start 46.9 76.16) (end 77.94 76.16) (width 0.12) (layer "F.Cu") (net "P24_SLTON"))
 (segment (start 46.9 99.375) (end 46.9 76.16) (width 0.12) (layer "F.Cu") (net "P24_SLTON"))
 (segment (start 77.94 76.16) (end 77.94 78.96) (width 0.12) (layer "F.Cu") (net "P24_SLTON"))
 (segment (start 63.97 97.45) (end 63.97 99.375) (width 0.12) (layer "F.Cu") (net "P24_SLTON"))
 (segment (start 63.97 99.375) (end 46.9 99.375) (width 0.12) (layer "F.Cu") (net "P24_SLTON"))
 (segment (start 65.239999 96.18) (end 65.239999 89.2) (width 0.25) (layer "F.Cu") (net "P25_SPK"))
 (segment (start 65.239999 89.2) (end 80.48 89.2) (width 0.25) (layer "F.Cu") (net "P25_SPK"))
 (segment (start 80.48 89.2) (end 80.48 81.5) (width 0.25) (layer "F.Cu") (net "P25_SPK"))
 (segment (start 46.6 99.61) (end 46.6 75.86) (width 0.12) (layer "B.Cu") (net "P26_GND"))
 (segment (start 65.239999 99.61) (end 46.6 99.61) (width 0.12) (layer "B.Cu") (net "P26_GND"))
 (segment (start 46.6 75.86) (end 80.48 75.86) (width 0.12) (layer "B.Cu") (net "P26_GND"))
 (segment (start 80.48 75.86) (end 80.48 78.96) (width 0.12) (layer "B.Cu") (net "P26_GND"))
 (segment (start 65.239999 97.45) (end 65.239999 99.61) (width 0.12) (layer "B.Cu") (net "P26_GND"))
 (segment (start 66.51 89.7) (end 83.02 89.7) (width 0.25) (layer "F.Cu") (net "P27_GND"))
 (segment (start 83.02 89.7) (end 83.02 81.5) (width 0.25) (layer "F.Cu") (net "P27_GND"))
 (segment (start 66.51 96.18) (end 66.51 89.7) (width 0.25) (layer "F.Cu") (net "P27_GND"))
 (segment (start 66.51 99.375) (end 113.91 99.375) (width 0.12) (layer "F.Cu") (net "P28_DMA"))
 (segment (start 113.91 76.16) (end 83.02 76.16) (width 0.12) (layer "F.Cu") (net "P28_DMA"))
 (segment (start 66.51 97.45) (end 66.51 99.375) (width 0.12) (layer "F.Cu") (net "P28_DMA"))
 (segment (start 113.91 99.375) (end 113.91 76.16) (width 0.12) (layer "F.Cu") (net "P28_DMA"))
 (segment (start 83.02 76.16) (end 83.02 78.96) (width 0.12) (layer "F.Cu") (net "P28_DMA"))
 (segment (start 67.78 96.18) (end 67.78 90.2) (width 0.25) (layer "F.Cu") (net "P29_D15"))
 (segment (start 85.56 90.2) (end 85.56 81.5) (width 0.25) (layer "F.Cu") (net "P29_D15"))
 (segment (start 67.78 90.2) (end 85.56 90.2) (width 0.25) (layer "F.Cu") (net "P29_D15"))
 (segment (start 113.91 76.16) (end 85.56 76.16) (width 0.12) (layer "B.Cu") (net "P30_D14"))
 (segment (start 85.56 76.16) (end 85.56 78.96) (width 0.12) (layer "B.Cu") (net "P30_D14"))
 (segment (start 67.78 99.375) (end 113.91 99.375) (width 0.12) (layer "B.Cu") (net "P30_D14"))
 (segment (start 113.91 99.375) (end 113.91 76.16) (width 0.12) (layer "B.Cu") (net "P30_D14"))
 (segment (start 67.78 97.45) (end 67.78 99.375) (width 0.12) (layer "B.Cu") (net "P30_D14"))
 (segment (start 69.05 96.18) (end 69.05 90.7) (width 0.25) (layer "F.Cu") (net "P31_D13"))
 (segment (start 69.05 90.7) (end 88.1 90.7) (width 0.25) (layer "F.Cu") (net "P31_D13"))
 (segment (start 88.1 90.7) (end 88.1 81.5) (width 0.25) (layer "F.Cu") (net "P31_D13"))
 (segment (start 69.05 97.45) (end 69.05 99.14) (width 0.12) (layer "F.Cu") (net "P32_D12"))
 (segment (start 88.1 76.46) (end 88.1 78.96) (width 0.12) (layer "F.Cu") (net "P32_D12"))
 (segment (start 69.05 99.14) (end 113.61 99.14) (width 0.12) (layer "F.Cu") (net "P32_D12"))
 (segment (start 113.61 76.46) (end 88.1 76.46) (width 0.12) (layer "F.Cu") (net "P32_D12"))
 (segment (start 113.61 99.14) (end 113.61 76.46) (width 0.12) (layer "F.Cu") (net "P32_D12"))
 (segment (start 90.64 91.2) (end 90.64 81.5) (width 0.25) (layer "F.Cu") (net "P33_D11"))
 (segment (start 70.32 91.2) (end 90.64 91.2) (width 0.25) (layer "F.Cu") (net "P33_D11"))
 (segment (start 70.32 96.18) (end 70.32 91.2) (width 0.25) (layer "F.Cu") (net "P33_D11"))
 (segment (start 113.61 99.14) (end 113.61 76.46) (width 0.12) (layer "B.Cu") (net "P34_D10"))
 (segment (start 113.61 76.46) (end 90.64 76.46) (width 0.12) (layer "B.Cu") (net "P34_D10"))
 (segment (start 70.32 97.45) (end 70.32 99.14) (width 0.12) (layer "B.Cu") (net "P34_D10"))
 (segment (start 70.32 99.14) (end 113.61 99.14) (width 0.12) (layer "B.Cu") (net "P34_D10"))
 (segment (start 90.64 76.46) (end 90.64 78.96) (width 0.12) (layer "B.Cu") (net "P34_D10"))
 (segment (start 93.18 91.7) (end 93.18 81.5) (width 0.25) (layer "F.Cu") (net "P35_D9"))
 (segment (start 71.59 91.7) (end 93.18 91.7) (width 0.25) (layer "F.Cu") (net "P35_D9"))
 (segment (start 71.59 96.18) (end 71.59 91.7) (width 0.25) (layer "F.Cu") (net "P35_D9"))
 (segment (start 93.18 76.759999) (end 93.18 78.96) (width 0.12) (layer "F.Cu") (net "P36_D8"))
 (segment (start 113.31 98.905) (end 113.31 76.759999) (width 0.12) (layer "F.Cu") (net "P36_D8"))
 (segment (start 113.31 76.759999) (end 93.18 76.759999) (width 0.12) (layer "F.Cu") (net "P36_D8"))
 (segment (start 71.59 98.905) (end 113.31 98.905) (width 0.12) (layer "F.Cu") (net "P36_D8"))
 (segment (start 71.59 97.45) (end 71.59 98.905) (width 0.12) (layer "F.Cu") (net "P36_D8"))
 (segment (start 72.86 92.2) (end 95.72 92.2) (width 0.25) (layer "F.Cu") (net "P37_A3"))
 (segment (start 95.72 92.2) (end 95.72 81.5) (width 0.25) (layer "F.Cu") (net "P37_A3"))
 (segment (start 72.86 96.18) (end 72.86 92.2) (width 0.25) (layer "F.Cu") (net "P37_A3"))
 (segment (start 113.31 76.759999) (end 95.72 76.759999) (width 0.12) (layer "B.Cu") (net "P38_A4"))
 (segment (start 95.72 76.759999) (end 95.72 78.96) (width 0.12) (layer "B.Cu") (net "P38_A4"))
 (segment (start 72.86 98.905) (end 113.31 98.905) (width 0.12) (layer "B.Cu") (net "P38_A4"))
 (segment (start 113.31 98.905) (end 113.31 76.759999) (width 0.12) (layer "B.Cu") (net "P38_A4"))
 (segment (start 72.86 97.45) (end 72.86 98.905) (width 0.12) (layer "B.Cu") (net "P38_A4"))
 (segment (start 74.13 96.18) (end 74.13 92.7) (width 0.25) (layer "F.Cu") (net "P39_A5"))
 (segment (start 98.259999 92.7) (end 98.259999 81.5) (width 0.25) (layer "F.Cu") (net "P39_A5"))
 (segment (start 74.13 92.7) (end 98.259999 92.7) (width 0.25) (layer "F.Cu") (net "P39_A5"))
 (segment (start 98.259999 77.06) (end 98.259999 78.96) (width 0.12) (layer "F.Cu") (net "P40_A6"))
 (segment (start 74.13 97.45) (end 74.13 98.67) (width 0.12) (layer "F.Cu") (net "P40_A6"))
 (segment (start 113.009999 77.06) (end 98.259999 77.06) (width 0.12) (layer "F.Cu") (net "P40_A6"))
 (segment (start 113.009999 98.67) (end 113.009999 77.06) (width 0.12) (layer "F.Cu") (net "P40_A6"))
 (segment (start 74.13 98.67) (end 113.009999 98.67) (width 0.12) (layer "F.Cu") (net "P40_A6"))
 (segment (start 75.4 93.2) (end 100.8 93.2) (width 0.25) (layer "F.Cu") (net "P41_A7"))
 (segment (start 100.8 93.2) (end 100.8 81.5) (width 0.25) (layer "F.Cu") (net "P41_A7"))
 (segment (start 75.4 96.18) (end 75.4 93.2) (width 0.25) (layer "F.Cu") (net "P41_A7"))
 (segment (start 75.4 97.45) (end 75.4 98.67) (width 0.12) (layer "B.Cu") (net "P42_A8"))
 (segment (start 100.8 77.06) (end 100.8 78.96) (width 0.12) (layer "B.Cu") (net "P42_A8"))
 (segment (start 75.4 98.67) (end 113.009999 98.67) (width 0.12) (layer "B.Cu") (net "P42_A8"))
 (segment (start 113.009999 77.06) (end 100.8 77.06) (width 0.12) (layer "B.Cu") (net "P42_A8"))
 (segment (start 113.009999 98.67) (end 113.009999 77.06) (width 0.12) (layer "B.Cu") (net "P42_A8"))
 (segment (start 76.67 93.7) (end 103.34 93.7) (width 0.25) (layer "F.Cu") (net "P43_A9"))
 (segment (start 76.67 96.18) (end 76.67 93.7) (width 0.25) (layer "F.Cu") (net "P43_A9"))
 (segment (start 103.34 93.7) (end 103.34 81.5) (width 0.25) (layer "F.Cu") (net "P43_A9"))
 (segment (start 76.67 97.45) (end 76.67 98.435) (width 0.12) (layer "F.Cu") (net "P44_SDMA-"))
 (segment (start 103.34 77.36) (end 103.34 78.96) (width 0.12) (layer "F.Cu") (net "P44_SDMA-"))
 (segment (start 76.67 98.435) (end 112.71 98.435) (width 0.12) (layer "F.Cu") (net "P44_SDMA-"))
 (segment (start 112.71 77.36) (end 103.34 77.36) (width 0.12) (layer "F.Cu") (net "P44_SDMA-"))
 (segment (start 112.71 98.435) (end 112.71 77.36) (width 0.12) (layer "F.Cu") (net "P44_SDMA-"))
 (segment (start 105.88 94.2) (end 105.88 81.5) (width 0.25) (layer "F.Cu") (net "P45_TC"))
 (segment (start 77.94 94.2) (end 105.88 94.2) (width 0.25) (layer "F.Cu") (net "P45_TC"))
 (segment (start 77.94 96.18) (end 77.94 94.2) (width 0.25) (layer "F.Cu") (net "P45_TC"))
 (segment (start 77.94 97.45) (end 77.94 98.435) (width 0.12) (layer "B.Cu") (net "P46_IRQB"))
 (segment (start 77.94 98.435) (end 112.71 98.435) (width 0.12) (layer "B.Cu") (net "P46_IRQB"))
 (segment (start 112.71 77.36) (end 105.88 77.36) (width 0.12) (layer "B.Cu") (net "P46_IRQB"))
 (segment (start 112.71 98.435) (end 112.71 77.36) (width 0.12) (layer "B.Cu") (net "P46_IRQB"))
 (segment (start 105.88 77.36) (end 105.88 78.96) (width 0.12) (layer "B.Cu") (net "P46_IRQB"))
 (segment (start 79.21 96.18) (end 79.21 94.7) (width 0.25) (layer "F.Cu") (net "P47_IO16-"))
 (segment (start 108.42 94.7) (end 108.42 81.5) (width 0.25) (layer "F.Cu") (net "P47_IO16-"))
 (segment (start 79.21 94.7) (end 108.42 94.7) (width 0.25) (layer "F.Cu") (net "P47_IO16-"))
 (segment (start 112.41 77.66) (end 108.42 77.66) (width 0.12) (layer "F.Cu") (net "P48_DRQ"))
 (segment (start 108.42 77.66) (end 108.42 78.96) (width 0.12) (layer "F.Cu") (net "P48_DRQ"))
 (segment (start 79.21 98.2) (end 112.41 98.2) (width 0.12) (layer "F.Cu") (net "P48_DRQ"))
 (segment (start 112.41 98.2) (end 112.41 77.66) (width 0.12) (layer "F.Cu") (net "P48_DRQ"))
 (segment (start 79.21 97.45) (end 79.21 98.2) (width 0.12) (layer "F.Cu") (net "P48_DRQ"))
 (segment (start 80.48 95.2) (end 110.96 95.2) (width 0.25) (layer "F.Cu") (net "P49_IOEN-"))
 (segment (start 80.48 96.18) (end 80.48 95.2) (width 0.25) (layer "F.Cu") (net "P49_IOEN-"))
 (segment (start 110.96 95.2) (end 110.96 81.5) (width 0.25) (layer "F.Cu") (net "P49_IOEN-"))
 (segment (start 110.96 77.66) (end 110.96 78.96) (width 0.12) (layer "B.Cu") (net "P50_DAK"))
 (segment (start 80.48 98.2) (end 112.41 98.2) (width 0.12) (layer "B.Cu") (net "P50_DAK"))
 (segment (start 80.48 97.45) (end 80.48 98.2) (width 0.12) (layer "B.Cu") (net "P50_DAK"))
 (segment (start 112.41 98.2) (end 112.41 77.66) (width 0.12) (layer "B.Cu") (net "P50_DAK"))
 (segment (start 112.41 77.66) (end 110.96 77.66) (width 0.12) (layer "B.Cu") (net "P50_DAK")))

